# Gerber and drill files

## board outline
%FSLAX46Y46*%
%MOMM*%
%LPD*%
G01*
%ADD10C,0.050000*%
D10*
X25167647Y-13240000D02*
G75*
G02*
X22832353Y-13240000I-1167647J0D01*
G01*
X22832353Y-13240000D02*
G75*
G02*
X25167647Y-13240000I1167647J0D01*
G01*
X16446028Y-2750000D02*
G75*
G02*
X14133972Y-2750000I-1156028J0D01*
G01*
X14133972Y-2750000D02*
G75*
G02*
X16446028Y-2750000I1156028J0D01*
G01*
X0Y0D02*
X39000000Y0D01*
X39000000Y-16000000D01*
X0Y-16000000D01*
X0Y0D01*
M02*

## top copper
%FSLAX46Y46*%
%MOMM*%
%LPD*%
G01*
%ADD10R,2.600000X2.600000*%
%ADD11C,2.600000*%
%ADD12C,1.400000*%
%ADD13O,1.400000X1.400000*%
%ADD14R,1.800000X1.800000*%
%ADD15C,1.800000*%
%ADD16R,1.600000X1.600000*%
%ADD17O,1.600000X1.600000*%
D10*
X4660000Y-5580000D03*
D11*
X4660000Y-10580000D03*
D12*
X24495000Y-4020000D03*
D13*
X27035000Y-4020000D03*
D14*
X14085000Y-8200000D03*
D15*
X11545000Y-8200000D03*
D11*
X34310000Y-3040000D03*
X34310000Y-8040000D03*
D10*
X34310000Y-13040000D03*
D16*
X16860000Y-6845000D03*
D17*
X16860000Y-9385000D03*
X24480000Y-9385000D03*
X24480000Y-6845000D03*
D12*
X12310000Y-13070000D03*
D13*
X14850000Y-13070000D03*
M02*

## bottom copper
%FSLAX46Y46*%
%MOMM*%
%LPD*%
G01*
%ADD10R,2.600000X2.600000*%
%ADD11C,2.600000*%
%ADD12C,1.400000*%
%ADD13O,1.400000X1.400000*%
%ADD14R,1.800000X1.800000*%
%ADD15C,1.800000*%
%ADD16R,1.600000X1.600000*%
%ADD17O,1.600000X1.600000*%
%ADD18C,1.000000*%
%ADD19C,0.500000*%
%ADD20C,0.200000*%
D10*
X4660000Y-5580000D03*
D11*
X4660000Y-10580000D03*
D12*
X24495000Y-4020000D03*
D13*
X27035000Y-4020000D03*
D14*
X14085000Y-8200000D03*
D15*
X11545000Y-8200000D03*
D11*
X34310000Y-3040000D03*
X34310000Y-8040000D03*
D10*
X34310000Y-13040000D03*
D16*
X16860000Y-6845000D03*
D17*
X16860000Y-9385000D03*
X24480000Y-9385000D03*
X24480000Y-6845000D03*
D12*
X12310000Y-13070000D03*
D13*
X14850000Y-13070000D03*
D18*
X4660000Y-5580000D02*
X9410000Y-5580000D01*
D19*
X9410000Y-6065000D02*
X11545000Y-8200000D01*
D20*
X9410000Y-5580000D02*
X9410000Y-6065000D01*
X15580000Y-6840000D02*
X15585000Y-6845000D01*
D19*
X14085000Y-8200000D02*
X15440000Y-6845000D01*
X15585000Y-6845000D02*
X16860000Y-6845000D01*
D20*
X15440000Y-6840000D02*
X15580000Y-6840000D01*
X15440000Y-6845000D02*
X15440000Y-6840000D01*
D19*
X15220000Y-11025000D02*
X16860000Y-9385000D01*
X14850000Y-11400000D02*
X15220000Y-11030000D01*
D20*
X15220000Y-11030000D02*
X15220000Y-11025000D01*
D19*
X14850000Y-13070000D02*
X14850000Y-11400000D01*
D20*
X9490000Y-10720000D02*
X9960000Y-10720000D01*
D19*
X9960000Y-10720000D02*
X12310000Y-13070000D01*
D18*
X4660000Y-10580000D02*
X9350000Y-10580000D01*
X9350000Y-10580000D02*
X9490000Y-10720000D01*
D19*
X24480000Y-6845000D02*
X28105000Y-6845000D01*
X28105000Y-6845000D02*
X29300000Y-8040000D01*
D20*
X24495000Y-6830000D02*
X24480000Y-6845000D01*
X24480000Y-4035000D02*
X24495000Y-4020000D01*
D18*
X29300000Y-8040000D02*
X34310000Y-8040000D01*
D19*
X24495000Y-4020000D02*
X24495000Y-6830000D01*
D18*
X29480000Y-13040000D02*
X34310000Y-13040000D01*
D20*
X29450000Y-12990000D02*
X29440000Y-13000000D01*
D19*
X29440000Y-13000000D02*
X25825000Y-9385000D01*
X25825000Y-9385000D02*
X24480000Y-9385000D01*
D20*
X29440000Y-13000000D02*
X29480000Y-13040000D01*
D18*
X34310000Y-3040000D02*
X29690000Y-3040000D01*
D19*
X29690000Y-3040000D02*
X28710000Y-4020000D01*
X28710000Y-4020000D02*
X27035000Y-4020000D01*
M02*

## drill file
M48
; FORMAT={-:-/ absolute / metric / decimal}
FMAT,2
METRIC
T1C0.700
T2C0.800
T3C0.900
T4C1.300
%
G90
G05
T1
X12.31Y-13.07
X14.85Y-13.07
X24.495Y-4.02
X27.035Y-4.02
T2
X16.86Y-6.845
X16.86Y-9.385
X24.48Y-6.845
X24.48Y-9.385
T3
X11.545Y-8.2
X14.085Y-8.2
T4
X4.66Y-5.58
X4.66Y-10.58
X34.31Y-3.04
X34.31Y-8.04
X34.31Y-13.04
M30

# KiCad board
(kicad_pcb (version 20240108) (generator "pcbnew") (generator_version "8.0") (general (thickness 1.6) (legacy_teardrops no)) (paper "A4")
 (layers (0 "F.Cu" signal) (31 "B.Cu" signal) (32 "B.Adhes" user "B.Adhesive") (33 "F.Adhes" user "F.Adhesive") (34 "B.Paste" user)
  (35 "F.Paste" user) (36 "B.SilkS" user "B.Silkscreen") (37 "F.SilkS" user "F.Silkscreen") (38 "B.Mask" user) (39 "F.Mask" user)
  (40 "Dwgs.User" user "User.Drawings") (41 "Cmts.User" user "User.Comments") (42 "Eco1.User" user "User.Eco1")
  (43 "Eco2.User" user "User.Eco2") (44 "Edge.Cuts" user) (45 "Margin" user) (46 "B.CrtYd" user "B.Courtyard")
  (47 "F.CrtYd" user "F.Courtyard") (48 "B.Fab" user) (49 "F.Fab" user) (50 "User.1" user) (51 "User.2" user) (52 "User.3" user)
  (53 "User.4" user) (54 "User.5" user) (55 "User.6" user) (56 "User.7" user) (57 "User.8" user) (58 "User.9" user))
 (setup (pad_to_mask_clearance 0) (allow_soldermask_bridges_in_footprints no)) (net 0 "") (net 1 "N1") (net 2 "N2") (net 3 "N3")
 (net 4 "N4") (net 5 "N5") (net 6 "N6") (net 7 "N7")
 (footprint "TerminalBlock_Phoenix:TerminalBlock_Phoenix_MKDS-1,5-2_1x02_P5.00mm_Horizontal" (layer "F.Cu") (at 4.66 5.58 -90)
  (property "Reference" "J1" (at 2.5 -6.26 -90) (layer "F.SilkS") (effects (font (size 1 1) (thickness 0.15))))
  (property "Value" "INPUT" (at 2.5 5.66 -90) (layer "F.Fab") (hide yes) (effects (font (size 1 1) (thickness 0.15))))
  (pad "1" thru_hole rect (at 0 0 270) (size 2.6 2.6) (drill 1.3) (layers "*.Cu" "*.Mask") (remove_unused_layers no) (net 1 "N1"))
  (pad "2" thru_hole circle (at 5 0 270) (size 2.6 2.6) (drill 1.3) (layers "*.Cu" "*.Mask") (remove_unused_layers no) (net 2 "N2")))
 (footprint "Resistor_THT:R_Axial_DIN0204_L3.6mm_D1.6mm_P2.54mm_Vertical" (layer "F.Cu") (at 24.495 4.02)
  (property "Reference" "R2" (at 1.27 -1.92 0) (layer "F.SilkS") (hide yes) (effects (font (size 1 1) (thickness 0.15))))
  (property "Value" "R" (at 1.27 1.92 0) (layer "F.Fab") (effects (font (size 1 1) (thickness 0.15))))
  (pad "1" thru_hole circle (at 0 0) (size 1.4 1.4) (drill 0.7) (layers "*.Cu" "*.Mask") (remove_unused_layers no) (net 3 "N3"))
  (pad "2" thru_hole oval (at 2.54 0) (size 1.4 1.4) (drill 0.7) (layers "*.Cu" "*.Mask") (remove_unused_layers no) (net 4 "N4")))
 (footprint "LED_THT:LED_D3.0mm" (layer "F.Cu") (at 14.085 8.2 180)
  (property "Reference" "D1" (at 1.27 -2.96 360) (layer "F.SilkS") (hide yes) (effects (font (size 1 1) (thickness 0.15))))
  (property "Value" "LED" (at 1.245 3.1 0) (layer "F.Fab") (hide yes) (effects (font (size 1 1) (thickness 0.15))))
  (pad "1" thru_hole rect (at 0 0 180) (size 1.8 1.8) (drill 0.9) (layers "*.Cu" "*.Mask") (remove_unused_layers no) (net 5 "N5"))
  (pad "2" thru_hole circle (at 2.54 0 180) (size 1.8 1.8) (drill 0.9) (layers "*.Cu" "*.Mask") (remove_unused_layers no) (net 1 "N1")))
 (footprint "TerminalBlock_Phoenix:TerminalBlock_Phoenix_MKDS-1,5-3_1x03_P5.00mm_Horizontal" (layer "F.Cu") (at 34.31 13.04 90)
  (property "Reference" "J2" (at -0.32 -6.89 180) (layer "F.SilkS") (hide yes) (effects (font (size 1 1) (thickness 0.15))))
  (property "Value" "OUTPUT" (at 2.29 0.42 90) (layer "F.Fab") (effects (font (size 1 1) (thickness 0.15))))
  (pad "1" thru_hole circle (at 10 0 90) (size 2.6 2.6) (drill 1.3) (layers "*.Cu" "*.Mask") (remove_unused_layers no) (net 4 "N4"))
  (pad "2" thru_hole circle (at 5 0 90) (size 2.6 2.6) (drill 1.3) (layers "*.Cu" "*.Mask") (remove_unused_layers no) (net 3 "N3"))
  (pad "3" thru_hole rect (at 0 0 90) (size 2.6 2.6) (drill 1.3) (layers "*.Cu" "*.Mask") (remove_unused_layers no) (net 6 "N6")))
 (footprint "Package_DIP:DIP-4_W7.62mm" (layer "F.Cu") (at 16.86 6.845)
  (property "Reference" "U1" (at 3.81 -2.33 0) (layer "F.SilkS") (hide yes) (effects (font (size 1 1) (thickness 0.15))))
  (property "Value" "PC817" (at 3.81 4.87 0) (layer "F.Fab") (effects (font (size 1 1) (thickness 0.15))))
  (pad "1" thru_hole rect (at 0 0) (size 1.6 1.6) (drill 0.8) (layers "*.Cu" "*.Mask") (remove_unused_layers no) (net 5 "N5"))
  (pad "2" thru_hole oval (at 0 2.54) (size 1.6 1.6) (drill 0.8) (layers "*.Cu" "*.Mask") (remove_unused_layers no) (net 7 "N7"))
  (pad "3" thru_hole oval (at 7.62 2.54) (size 1.6 1.6) (drill 0.8) (layers "*.Cu" "*.Mask") (remove_unused_layers no) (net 6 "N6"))
  (pad "4" thru_hole oval (at 7.62 0) (size 1.6 1.6) (drill 0.8) (layers "*.Cu" "*.Mask") (remove_unused_layers no) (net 3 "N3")))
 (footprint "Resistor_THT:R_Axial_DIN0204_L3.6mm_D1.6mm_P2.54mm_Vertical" (layer "F.Cu") (at 12.31 13.07)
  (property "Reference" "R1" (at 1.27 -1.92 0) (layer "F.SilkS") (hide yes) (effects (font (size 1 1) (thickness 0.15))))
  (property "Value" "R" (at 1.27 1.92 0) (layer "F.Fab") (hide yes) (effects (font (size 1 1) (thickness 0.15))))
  (pad "1" thru_hole circle (at 0 0) (size 1.4 1.4) (drill 0.7) (layers "*.Cu" "*.Mask") (remove_unused_layers no) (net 2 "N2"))
  (pad "2" thru_hole oval (at 2.54 0) (size 1.4 1.4) (drill 0.7) (layers "*.Cu" "*.Mask") (remove_unused_layers no) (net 7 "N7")))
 (gr_circle (center 24 13.24) (end 25.167647 13.24) (stroke (width 0.05) (type default)) (fill none) (layer "Edge.Cuts"))
 (gr_circle (center 15.29 2.75) (end 16.446028 2.75) (stroke (width 0.05) (type default)) (fill none) (layer "Edge.Cuts"))
 (gr_rect (start 0 0) (end 39 16) (stroke (width 0.05) (type default)) (fill none) (layer "Edge.Cuts"))
 (segment (start 4.66 5.58) (end 9.41 5.58) (width 1) (layer "B.Cu") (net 1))
 (segment (start 9.41 6.065) (end 11.545 8.2) (width 0.5) (layer "B.Cu") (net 1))
 (segment (start 9.41 5.58) (end 9.41 6.065) (width 0.2) (layer "B.Cu") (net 1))
 (segment (start 15.58 6.84) (end 15.585 6.845) (width 0.2) (layer "B.Cu") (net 5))
 (segment (start 14.085 8.2) (end 15.44 6.845) (width 0.5) (layer "B.Cu") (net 5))
 (segment (start 15.585 6.845) (end 16.86 6.845) (width 0.5) (layer "B.Cu") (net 5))
 (segment (start 15.44 6.84) (end 15.58 6.84) (width 0.2) (layer "B.Cu") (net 5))
 (segment (start 15.44 6.845) (end 15.44 6.84) (width 0.2) (layer "B.Cu") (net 5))
 (segment (start 15.22 11.025) (end 16.86 9.385) (width 0.5) (layer "B.Cu") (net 7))
 (segment (start 14.85 11.4) (end 15.22 11.03) (width 0.5) (layer "B.Cu") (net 7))
 (segment (start 15.22 11.03) (end 15.22 11.025) (width 0.2) (layer "B.Cu") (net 7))
 (segment (start 14.85 13.07) (end 14.85 11.4) (width 0.5) (layer "B.Cu") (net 7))
 (segment (start 9.49 10.72) (end 9.96 10.72) (width 0.2) (layer "B.Cu") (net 2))
 (segment (start 9.96 10.72) (end 12.31 13.07) (width 0.5) (layer "B.Cu") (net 2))
 (segment (start 4.66 10.58) (end 9.35 10.58) (width 1) (layer "B.Cu") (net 2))
 (segment (start 9.35 10.58) (end 9.49 10.72) (width 1) (layer "B.Cu") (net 2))
 (segment (start 24.48 6.845) (end 28.105 6.845) (width 0.5) (layer "B.Cu") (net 3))
 (segment (start 28.105 6.845) (end 29.3 8.04) (width 0.5) (layer "B.Cu") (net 3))
 (segment (start 24.495 6.83) (end 24.48 6.845) (width 0.2) (layer "B.Cu") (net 3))
 (segment (start 24.48 4.035) (end 24.495 4.02) (width 0.2) (layer "B.Cu") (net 3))
 (segment (start 29.3 8.04) (end 34.31 8.04) (width 1) (layer "B.Cu") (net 3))
 (segment (start 24.495 4.02) (end 24.495 6.83) (width 0.5) (layer "B.Cu") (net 3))
 (segment (start 29.48 13.04) (end 34.31 13.04) (width 1) (layer "B.Cu") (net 6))
 (segment (start 29.45 12.99) (end 29.44 13) (width 0.2) (layer "B.Cu") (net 6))
 (segment (start 29.44 13) (end 25.825 9.385) (width 0.5) (layer "B.Cu") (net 6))
 (segment (start 25.825 9.385) (end 24.48 9.385) (width 0.5) (layer "B.Cu") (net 6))
 (segment (start 29.44 13) (end 29.48 13.04) (width 0.2) (layer "B.Cu") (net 6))
 (segment (start 34.31 3.04) (end 29.69 3.04) (width 1) (layer "B.Cu") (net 4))
 (segment (start 29.69 3.04) (end 28.71 4.02) (width 0.5) (layer "B.Cu") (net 4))
 (segment (start 28.71 4.02) (end 27.035 4.02) (width 0.5) (layer "B.Cu") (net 4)))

